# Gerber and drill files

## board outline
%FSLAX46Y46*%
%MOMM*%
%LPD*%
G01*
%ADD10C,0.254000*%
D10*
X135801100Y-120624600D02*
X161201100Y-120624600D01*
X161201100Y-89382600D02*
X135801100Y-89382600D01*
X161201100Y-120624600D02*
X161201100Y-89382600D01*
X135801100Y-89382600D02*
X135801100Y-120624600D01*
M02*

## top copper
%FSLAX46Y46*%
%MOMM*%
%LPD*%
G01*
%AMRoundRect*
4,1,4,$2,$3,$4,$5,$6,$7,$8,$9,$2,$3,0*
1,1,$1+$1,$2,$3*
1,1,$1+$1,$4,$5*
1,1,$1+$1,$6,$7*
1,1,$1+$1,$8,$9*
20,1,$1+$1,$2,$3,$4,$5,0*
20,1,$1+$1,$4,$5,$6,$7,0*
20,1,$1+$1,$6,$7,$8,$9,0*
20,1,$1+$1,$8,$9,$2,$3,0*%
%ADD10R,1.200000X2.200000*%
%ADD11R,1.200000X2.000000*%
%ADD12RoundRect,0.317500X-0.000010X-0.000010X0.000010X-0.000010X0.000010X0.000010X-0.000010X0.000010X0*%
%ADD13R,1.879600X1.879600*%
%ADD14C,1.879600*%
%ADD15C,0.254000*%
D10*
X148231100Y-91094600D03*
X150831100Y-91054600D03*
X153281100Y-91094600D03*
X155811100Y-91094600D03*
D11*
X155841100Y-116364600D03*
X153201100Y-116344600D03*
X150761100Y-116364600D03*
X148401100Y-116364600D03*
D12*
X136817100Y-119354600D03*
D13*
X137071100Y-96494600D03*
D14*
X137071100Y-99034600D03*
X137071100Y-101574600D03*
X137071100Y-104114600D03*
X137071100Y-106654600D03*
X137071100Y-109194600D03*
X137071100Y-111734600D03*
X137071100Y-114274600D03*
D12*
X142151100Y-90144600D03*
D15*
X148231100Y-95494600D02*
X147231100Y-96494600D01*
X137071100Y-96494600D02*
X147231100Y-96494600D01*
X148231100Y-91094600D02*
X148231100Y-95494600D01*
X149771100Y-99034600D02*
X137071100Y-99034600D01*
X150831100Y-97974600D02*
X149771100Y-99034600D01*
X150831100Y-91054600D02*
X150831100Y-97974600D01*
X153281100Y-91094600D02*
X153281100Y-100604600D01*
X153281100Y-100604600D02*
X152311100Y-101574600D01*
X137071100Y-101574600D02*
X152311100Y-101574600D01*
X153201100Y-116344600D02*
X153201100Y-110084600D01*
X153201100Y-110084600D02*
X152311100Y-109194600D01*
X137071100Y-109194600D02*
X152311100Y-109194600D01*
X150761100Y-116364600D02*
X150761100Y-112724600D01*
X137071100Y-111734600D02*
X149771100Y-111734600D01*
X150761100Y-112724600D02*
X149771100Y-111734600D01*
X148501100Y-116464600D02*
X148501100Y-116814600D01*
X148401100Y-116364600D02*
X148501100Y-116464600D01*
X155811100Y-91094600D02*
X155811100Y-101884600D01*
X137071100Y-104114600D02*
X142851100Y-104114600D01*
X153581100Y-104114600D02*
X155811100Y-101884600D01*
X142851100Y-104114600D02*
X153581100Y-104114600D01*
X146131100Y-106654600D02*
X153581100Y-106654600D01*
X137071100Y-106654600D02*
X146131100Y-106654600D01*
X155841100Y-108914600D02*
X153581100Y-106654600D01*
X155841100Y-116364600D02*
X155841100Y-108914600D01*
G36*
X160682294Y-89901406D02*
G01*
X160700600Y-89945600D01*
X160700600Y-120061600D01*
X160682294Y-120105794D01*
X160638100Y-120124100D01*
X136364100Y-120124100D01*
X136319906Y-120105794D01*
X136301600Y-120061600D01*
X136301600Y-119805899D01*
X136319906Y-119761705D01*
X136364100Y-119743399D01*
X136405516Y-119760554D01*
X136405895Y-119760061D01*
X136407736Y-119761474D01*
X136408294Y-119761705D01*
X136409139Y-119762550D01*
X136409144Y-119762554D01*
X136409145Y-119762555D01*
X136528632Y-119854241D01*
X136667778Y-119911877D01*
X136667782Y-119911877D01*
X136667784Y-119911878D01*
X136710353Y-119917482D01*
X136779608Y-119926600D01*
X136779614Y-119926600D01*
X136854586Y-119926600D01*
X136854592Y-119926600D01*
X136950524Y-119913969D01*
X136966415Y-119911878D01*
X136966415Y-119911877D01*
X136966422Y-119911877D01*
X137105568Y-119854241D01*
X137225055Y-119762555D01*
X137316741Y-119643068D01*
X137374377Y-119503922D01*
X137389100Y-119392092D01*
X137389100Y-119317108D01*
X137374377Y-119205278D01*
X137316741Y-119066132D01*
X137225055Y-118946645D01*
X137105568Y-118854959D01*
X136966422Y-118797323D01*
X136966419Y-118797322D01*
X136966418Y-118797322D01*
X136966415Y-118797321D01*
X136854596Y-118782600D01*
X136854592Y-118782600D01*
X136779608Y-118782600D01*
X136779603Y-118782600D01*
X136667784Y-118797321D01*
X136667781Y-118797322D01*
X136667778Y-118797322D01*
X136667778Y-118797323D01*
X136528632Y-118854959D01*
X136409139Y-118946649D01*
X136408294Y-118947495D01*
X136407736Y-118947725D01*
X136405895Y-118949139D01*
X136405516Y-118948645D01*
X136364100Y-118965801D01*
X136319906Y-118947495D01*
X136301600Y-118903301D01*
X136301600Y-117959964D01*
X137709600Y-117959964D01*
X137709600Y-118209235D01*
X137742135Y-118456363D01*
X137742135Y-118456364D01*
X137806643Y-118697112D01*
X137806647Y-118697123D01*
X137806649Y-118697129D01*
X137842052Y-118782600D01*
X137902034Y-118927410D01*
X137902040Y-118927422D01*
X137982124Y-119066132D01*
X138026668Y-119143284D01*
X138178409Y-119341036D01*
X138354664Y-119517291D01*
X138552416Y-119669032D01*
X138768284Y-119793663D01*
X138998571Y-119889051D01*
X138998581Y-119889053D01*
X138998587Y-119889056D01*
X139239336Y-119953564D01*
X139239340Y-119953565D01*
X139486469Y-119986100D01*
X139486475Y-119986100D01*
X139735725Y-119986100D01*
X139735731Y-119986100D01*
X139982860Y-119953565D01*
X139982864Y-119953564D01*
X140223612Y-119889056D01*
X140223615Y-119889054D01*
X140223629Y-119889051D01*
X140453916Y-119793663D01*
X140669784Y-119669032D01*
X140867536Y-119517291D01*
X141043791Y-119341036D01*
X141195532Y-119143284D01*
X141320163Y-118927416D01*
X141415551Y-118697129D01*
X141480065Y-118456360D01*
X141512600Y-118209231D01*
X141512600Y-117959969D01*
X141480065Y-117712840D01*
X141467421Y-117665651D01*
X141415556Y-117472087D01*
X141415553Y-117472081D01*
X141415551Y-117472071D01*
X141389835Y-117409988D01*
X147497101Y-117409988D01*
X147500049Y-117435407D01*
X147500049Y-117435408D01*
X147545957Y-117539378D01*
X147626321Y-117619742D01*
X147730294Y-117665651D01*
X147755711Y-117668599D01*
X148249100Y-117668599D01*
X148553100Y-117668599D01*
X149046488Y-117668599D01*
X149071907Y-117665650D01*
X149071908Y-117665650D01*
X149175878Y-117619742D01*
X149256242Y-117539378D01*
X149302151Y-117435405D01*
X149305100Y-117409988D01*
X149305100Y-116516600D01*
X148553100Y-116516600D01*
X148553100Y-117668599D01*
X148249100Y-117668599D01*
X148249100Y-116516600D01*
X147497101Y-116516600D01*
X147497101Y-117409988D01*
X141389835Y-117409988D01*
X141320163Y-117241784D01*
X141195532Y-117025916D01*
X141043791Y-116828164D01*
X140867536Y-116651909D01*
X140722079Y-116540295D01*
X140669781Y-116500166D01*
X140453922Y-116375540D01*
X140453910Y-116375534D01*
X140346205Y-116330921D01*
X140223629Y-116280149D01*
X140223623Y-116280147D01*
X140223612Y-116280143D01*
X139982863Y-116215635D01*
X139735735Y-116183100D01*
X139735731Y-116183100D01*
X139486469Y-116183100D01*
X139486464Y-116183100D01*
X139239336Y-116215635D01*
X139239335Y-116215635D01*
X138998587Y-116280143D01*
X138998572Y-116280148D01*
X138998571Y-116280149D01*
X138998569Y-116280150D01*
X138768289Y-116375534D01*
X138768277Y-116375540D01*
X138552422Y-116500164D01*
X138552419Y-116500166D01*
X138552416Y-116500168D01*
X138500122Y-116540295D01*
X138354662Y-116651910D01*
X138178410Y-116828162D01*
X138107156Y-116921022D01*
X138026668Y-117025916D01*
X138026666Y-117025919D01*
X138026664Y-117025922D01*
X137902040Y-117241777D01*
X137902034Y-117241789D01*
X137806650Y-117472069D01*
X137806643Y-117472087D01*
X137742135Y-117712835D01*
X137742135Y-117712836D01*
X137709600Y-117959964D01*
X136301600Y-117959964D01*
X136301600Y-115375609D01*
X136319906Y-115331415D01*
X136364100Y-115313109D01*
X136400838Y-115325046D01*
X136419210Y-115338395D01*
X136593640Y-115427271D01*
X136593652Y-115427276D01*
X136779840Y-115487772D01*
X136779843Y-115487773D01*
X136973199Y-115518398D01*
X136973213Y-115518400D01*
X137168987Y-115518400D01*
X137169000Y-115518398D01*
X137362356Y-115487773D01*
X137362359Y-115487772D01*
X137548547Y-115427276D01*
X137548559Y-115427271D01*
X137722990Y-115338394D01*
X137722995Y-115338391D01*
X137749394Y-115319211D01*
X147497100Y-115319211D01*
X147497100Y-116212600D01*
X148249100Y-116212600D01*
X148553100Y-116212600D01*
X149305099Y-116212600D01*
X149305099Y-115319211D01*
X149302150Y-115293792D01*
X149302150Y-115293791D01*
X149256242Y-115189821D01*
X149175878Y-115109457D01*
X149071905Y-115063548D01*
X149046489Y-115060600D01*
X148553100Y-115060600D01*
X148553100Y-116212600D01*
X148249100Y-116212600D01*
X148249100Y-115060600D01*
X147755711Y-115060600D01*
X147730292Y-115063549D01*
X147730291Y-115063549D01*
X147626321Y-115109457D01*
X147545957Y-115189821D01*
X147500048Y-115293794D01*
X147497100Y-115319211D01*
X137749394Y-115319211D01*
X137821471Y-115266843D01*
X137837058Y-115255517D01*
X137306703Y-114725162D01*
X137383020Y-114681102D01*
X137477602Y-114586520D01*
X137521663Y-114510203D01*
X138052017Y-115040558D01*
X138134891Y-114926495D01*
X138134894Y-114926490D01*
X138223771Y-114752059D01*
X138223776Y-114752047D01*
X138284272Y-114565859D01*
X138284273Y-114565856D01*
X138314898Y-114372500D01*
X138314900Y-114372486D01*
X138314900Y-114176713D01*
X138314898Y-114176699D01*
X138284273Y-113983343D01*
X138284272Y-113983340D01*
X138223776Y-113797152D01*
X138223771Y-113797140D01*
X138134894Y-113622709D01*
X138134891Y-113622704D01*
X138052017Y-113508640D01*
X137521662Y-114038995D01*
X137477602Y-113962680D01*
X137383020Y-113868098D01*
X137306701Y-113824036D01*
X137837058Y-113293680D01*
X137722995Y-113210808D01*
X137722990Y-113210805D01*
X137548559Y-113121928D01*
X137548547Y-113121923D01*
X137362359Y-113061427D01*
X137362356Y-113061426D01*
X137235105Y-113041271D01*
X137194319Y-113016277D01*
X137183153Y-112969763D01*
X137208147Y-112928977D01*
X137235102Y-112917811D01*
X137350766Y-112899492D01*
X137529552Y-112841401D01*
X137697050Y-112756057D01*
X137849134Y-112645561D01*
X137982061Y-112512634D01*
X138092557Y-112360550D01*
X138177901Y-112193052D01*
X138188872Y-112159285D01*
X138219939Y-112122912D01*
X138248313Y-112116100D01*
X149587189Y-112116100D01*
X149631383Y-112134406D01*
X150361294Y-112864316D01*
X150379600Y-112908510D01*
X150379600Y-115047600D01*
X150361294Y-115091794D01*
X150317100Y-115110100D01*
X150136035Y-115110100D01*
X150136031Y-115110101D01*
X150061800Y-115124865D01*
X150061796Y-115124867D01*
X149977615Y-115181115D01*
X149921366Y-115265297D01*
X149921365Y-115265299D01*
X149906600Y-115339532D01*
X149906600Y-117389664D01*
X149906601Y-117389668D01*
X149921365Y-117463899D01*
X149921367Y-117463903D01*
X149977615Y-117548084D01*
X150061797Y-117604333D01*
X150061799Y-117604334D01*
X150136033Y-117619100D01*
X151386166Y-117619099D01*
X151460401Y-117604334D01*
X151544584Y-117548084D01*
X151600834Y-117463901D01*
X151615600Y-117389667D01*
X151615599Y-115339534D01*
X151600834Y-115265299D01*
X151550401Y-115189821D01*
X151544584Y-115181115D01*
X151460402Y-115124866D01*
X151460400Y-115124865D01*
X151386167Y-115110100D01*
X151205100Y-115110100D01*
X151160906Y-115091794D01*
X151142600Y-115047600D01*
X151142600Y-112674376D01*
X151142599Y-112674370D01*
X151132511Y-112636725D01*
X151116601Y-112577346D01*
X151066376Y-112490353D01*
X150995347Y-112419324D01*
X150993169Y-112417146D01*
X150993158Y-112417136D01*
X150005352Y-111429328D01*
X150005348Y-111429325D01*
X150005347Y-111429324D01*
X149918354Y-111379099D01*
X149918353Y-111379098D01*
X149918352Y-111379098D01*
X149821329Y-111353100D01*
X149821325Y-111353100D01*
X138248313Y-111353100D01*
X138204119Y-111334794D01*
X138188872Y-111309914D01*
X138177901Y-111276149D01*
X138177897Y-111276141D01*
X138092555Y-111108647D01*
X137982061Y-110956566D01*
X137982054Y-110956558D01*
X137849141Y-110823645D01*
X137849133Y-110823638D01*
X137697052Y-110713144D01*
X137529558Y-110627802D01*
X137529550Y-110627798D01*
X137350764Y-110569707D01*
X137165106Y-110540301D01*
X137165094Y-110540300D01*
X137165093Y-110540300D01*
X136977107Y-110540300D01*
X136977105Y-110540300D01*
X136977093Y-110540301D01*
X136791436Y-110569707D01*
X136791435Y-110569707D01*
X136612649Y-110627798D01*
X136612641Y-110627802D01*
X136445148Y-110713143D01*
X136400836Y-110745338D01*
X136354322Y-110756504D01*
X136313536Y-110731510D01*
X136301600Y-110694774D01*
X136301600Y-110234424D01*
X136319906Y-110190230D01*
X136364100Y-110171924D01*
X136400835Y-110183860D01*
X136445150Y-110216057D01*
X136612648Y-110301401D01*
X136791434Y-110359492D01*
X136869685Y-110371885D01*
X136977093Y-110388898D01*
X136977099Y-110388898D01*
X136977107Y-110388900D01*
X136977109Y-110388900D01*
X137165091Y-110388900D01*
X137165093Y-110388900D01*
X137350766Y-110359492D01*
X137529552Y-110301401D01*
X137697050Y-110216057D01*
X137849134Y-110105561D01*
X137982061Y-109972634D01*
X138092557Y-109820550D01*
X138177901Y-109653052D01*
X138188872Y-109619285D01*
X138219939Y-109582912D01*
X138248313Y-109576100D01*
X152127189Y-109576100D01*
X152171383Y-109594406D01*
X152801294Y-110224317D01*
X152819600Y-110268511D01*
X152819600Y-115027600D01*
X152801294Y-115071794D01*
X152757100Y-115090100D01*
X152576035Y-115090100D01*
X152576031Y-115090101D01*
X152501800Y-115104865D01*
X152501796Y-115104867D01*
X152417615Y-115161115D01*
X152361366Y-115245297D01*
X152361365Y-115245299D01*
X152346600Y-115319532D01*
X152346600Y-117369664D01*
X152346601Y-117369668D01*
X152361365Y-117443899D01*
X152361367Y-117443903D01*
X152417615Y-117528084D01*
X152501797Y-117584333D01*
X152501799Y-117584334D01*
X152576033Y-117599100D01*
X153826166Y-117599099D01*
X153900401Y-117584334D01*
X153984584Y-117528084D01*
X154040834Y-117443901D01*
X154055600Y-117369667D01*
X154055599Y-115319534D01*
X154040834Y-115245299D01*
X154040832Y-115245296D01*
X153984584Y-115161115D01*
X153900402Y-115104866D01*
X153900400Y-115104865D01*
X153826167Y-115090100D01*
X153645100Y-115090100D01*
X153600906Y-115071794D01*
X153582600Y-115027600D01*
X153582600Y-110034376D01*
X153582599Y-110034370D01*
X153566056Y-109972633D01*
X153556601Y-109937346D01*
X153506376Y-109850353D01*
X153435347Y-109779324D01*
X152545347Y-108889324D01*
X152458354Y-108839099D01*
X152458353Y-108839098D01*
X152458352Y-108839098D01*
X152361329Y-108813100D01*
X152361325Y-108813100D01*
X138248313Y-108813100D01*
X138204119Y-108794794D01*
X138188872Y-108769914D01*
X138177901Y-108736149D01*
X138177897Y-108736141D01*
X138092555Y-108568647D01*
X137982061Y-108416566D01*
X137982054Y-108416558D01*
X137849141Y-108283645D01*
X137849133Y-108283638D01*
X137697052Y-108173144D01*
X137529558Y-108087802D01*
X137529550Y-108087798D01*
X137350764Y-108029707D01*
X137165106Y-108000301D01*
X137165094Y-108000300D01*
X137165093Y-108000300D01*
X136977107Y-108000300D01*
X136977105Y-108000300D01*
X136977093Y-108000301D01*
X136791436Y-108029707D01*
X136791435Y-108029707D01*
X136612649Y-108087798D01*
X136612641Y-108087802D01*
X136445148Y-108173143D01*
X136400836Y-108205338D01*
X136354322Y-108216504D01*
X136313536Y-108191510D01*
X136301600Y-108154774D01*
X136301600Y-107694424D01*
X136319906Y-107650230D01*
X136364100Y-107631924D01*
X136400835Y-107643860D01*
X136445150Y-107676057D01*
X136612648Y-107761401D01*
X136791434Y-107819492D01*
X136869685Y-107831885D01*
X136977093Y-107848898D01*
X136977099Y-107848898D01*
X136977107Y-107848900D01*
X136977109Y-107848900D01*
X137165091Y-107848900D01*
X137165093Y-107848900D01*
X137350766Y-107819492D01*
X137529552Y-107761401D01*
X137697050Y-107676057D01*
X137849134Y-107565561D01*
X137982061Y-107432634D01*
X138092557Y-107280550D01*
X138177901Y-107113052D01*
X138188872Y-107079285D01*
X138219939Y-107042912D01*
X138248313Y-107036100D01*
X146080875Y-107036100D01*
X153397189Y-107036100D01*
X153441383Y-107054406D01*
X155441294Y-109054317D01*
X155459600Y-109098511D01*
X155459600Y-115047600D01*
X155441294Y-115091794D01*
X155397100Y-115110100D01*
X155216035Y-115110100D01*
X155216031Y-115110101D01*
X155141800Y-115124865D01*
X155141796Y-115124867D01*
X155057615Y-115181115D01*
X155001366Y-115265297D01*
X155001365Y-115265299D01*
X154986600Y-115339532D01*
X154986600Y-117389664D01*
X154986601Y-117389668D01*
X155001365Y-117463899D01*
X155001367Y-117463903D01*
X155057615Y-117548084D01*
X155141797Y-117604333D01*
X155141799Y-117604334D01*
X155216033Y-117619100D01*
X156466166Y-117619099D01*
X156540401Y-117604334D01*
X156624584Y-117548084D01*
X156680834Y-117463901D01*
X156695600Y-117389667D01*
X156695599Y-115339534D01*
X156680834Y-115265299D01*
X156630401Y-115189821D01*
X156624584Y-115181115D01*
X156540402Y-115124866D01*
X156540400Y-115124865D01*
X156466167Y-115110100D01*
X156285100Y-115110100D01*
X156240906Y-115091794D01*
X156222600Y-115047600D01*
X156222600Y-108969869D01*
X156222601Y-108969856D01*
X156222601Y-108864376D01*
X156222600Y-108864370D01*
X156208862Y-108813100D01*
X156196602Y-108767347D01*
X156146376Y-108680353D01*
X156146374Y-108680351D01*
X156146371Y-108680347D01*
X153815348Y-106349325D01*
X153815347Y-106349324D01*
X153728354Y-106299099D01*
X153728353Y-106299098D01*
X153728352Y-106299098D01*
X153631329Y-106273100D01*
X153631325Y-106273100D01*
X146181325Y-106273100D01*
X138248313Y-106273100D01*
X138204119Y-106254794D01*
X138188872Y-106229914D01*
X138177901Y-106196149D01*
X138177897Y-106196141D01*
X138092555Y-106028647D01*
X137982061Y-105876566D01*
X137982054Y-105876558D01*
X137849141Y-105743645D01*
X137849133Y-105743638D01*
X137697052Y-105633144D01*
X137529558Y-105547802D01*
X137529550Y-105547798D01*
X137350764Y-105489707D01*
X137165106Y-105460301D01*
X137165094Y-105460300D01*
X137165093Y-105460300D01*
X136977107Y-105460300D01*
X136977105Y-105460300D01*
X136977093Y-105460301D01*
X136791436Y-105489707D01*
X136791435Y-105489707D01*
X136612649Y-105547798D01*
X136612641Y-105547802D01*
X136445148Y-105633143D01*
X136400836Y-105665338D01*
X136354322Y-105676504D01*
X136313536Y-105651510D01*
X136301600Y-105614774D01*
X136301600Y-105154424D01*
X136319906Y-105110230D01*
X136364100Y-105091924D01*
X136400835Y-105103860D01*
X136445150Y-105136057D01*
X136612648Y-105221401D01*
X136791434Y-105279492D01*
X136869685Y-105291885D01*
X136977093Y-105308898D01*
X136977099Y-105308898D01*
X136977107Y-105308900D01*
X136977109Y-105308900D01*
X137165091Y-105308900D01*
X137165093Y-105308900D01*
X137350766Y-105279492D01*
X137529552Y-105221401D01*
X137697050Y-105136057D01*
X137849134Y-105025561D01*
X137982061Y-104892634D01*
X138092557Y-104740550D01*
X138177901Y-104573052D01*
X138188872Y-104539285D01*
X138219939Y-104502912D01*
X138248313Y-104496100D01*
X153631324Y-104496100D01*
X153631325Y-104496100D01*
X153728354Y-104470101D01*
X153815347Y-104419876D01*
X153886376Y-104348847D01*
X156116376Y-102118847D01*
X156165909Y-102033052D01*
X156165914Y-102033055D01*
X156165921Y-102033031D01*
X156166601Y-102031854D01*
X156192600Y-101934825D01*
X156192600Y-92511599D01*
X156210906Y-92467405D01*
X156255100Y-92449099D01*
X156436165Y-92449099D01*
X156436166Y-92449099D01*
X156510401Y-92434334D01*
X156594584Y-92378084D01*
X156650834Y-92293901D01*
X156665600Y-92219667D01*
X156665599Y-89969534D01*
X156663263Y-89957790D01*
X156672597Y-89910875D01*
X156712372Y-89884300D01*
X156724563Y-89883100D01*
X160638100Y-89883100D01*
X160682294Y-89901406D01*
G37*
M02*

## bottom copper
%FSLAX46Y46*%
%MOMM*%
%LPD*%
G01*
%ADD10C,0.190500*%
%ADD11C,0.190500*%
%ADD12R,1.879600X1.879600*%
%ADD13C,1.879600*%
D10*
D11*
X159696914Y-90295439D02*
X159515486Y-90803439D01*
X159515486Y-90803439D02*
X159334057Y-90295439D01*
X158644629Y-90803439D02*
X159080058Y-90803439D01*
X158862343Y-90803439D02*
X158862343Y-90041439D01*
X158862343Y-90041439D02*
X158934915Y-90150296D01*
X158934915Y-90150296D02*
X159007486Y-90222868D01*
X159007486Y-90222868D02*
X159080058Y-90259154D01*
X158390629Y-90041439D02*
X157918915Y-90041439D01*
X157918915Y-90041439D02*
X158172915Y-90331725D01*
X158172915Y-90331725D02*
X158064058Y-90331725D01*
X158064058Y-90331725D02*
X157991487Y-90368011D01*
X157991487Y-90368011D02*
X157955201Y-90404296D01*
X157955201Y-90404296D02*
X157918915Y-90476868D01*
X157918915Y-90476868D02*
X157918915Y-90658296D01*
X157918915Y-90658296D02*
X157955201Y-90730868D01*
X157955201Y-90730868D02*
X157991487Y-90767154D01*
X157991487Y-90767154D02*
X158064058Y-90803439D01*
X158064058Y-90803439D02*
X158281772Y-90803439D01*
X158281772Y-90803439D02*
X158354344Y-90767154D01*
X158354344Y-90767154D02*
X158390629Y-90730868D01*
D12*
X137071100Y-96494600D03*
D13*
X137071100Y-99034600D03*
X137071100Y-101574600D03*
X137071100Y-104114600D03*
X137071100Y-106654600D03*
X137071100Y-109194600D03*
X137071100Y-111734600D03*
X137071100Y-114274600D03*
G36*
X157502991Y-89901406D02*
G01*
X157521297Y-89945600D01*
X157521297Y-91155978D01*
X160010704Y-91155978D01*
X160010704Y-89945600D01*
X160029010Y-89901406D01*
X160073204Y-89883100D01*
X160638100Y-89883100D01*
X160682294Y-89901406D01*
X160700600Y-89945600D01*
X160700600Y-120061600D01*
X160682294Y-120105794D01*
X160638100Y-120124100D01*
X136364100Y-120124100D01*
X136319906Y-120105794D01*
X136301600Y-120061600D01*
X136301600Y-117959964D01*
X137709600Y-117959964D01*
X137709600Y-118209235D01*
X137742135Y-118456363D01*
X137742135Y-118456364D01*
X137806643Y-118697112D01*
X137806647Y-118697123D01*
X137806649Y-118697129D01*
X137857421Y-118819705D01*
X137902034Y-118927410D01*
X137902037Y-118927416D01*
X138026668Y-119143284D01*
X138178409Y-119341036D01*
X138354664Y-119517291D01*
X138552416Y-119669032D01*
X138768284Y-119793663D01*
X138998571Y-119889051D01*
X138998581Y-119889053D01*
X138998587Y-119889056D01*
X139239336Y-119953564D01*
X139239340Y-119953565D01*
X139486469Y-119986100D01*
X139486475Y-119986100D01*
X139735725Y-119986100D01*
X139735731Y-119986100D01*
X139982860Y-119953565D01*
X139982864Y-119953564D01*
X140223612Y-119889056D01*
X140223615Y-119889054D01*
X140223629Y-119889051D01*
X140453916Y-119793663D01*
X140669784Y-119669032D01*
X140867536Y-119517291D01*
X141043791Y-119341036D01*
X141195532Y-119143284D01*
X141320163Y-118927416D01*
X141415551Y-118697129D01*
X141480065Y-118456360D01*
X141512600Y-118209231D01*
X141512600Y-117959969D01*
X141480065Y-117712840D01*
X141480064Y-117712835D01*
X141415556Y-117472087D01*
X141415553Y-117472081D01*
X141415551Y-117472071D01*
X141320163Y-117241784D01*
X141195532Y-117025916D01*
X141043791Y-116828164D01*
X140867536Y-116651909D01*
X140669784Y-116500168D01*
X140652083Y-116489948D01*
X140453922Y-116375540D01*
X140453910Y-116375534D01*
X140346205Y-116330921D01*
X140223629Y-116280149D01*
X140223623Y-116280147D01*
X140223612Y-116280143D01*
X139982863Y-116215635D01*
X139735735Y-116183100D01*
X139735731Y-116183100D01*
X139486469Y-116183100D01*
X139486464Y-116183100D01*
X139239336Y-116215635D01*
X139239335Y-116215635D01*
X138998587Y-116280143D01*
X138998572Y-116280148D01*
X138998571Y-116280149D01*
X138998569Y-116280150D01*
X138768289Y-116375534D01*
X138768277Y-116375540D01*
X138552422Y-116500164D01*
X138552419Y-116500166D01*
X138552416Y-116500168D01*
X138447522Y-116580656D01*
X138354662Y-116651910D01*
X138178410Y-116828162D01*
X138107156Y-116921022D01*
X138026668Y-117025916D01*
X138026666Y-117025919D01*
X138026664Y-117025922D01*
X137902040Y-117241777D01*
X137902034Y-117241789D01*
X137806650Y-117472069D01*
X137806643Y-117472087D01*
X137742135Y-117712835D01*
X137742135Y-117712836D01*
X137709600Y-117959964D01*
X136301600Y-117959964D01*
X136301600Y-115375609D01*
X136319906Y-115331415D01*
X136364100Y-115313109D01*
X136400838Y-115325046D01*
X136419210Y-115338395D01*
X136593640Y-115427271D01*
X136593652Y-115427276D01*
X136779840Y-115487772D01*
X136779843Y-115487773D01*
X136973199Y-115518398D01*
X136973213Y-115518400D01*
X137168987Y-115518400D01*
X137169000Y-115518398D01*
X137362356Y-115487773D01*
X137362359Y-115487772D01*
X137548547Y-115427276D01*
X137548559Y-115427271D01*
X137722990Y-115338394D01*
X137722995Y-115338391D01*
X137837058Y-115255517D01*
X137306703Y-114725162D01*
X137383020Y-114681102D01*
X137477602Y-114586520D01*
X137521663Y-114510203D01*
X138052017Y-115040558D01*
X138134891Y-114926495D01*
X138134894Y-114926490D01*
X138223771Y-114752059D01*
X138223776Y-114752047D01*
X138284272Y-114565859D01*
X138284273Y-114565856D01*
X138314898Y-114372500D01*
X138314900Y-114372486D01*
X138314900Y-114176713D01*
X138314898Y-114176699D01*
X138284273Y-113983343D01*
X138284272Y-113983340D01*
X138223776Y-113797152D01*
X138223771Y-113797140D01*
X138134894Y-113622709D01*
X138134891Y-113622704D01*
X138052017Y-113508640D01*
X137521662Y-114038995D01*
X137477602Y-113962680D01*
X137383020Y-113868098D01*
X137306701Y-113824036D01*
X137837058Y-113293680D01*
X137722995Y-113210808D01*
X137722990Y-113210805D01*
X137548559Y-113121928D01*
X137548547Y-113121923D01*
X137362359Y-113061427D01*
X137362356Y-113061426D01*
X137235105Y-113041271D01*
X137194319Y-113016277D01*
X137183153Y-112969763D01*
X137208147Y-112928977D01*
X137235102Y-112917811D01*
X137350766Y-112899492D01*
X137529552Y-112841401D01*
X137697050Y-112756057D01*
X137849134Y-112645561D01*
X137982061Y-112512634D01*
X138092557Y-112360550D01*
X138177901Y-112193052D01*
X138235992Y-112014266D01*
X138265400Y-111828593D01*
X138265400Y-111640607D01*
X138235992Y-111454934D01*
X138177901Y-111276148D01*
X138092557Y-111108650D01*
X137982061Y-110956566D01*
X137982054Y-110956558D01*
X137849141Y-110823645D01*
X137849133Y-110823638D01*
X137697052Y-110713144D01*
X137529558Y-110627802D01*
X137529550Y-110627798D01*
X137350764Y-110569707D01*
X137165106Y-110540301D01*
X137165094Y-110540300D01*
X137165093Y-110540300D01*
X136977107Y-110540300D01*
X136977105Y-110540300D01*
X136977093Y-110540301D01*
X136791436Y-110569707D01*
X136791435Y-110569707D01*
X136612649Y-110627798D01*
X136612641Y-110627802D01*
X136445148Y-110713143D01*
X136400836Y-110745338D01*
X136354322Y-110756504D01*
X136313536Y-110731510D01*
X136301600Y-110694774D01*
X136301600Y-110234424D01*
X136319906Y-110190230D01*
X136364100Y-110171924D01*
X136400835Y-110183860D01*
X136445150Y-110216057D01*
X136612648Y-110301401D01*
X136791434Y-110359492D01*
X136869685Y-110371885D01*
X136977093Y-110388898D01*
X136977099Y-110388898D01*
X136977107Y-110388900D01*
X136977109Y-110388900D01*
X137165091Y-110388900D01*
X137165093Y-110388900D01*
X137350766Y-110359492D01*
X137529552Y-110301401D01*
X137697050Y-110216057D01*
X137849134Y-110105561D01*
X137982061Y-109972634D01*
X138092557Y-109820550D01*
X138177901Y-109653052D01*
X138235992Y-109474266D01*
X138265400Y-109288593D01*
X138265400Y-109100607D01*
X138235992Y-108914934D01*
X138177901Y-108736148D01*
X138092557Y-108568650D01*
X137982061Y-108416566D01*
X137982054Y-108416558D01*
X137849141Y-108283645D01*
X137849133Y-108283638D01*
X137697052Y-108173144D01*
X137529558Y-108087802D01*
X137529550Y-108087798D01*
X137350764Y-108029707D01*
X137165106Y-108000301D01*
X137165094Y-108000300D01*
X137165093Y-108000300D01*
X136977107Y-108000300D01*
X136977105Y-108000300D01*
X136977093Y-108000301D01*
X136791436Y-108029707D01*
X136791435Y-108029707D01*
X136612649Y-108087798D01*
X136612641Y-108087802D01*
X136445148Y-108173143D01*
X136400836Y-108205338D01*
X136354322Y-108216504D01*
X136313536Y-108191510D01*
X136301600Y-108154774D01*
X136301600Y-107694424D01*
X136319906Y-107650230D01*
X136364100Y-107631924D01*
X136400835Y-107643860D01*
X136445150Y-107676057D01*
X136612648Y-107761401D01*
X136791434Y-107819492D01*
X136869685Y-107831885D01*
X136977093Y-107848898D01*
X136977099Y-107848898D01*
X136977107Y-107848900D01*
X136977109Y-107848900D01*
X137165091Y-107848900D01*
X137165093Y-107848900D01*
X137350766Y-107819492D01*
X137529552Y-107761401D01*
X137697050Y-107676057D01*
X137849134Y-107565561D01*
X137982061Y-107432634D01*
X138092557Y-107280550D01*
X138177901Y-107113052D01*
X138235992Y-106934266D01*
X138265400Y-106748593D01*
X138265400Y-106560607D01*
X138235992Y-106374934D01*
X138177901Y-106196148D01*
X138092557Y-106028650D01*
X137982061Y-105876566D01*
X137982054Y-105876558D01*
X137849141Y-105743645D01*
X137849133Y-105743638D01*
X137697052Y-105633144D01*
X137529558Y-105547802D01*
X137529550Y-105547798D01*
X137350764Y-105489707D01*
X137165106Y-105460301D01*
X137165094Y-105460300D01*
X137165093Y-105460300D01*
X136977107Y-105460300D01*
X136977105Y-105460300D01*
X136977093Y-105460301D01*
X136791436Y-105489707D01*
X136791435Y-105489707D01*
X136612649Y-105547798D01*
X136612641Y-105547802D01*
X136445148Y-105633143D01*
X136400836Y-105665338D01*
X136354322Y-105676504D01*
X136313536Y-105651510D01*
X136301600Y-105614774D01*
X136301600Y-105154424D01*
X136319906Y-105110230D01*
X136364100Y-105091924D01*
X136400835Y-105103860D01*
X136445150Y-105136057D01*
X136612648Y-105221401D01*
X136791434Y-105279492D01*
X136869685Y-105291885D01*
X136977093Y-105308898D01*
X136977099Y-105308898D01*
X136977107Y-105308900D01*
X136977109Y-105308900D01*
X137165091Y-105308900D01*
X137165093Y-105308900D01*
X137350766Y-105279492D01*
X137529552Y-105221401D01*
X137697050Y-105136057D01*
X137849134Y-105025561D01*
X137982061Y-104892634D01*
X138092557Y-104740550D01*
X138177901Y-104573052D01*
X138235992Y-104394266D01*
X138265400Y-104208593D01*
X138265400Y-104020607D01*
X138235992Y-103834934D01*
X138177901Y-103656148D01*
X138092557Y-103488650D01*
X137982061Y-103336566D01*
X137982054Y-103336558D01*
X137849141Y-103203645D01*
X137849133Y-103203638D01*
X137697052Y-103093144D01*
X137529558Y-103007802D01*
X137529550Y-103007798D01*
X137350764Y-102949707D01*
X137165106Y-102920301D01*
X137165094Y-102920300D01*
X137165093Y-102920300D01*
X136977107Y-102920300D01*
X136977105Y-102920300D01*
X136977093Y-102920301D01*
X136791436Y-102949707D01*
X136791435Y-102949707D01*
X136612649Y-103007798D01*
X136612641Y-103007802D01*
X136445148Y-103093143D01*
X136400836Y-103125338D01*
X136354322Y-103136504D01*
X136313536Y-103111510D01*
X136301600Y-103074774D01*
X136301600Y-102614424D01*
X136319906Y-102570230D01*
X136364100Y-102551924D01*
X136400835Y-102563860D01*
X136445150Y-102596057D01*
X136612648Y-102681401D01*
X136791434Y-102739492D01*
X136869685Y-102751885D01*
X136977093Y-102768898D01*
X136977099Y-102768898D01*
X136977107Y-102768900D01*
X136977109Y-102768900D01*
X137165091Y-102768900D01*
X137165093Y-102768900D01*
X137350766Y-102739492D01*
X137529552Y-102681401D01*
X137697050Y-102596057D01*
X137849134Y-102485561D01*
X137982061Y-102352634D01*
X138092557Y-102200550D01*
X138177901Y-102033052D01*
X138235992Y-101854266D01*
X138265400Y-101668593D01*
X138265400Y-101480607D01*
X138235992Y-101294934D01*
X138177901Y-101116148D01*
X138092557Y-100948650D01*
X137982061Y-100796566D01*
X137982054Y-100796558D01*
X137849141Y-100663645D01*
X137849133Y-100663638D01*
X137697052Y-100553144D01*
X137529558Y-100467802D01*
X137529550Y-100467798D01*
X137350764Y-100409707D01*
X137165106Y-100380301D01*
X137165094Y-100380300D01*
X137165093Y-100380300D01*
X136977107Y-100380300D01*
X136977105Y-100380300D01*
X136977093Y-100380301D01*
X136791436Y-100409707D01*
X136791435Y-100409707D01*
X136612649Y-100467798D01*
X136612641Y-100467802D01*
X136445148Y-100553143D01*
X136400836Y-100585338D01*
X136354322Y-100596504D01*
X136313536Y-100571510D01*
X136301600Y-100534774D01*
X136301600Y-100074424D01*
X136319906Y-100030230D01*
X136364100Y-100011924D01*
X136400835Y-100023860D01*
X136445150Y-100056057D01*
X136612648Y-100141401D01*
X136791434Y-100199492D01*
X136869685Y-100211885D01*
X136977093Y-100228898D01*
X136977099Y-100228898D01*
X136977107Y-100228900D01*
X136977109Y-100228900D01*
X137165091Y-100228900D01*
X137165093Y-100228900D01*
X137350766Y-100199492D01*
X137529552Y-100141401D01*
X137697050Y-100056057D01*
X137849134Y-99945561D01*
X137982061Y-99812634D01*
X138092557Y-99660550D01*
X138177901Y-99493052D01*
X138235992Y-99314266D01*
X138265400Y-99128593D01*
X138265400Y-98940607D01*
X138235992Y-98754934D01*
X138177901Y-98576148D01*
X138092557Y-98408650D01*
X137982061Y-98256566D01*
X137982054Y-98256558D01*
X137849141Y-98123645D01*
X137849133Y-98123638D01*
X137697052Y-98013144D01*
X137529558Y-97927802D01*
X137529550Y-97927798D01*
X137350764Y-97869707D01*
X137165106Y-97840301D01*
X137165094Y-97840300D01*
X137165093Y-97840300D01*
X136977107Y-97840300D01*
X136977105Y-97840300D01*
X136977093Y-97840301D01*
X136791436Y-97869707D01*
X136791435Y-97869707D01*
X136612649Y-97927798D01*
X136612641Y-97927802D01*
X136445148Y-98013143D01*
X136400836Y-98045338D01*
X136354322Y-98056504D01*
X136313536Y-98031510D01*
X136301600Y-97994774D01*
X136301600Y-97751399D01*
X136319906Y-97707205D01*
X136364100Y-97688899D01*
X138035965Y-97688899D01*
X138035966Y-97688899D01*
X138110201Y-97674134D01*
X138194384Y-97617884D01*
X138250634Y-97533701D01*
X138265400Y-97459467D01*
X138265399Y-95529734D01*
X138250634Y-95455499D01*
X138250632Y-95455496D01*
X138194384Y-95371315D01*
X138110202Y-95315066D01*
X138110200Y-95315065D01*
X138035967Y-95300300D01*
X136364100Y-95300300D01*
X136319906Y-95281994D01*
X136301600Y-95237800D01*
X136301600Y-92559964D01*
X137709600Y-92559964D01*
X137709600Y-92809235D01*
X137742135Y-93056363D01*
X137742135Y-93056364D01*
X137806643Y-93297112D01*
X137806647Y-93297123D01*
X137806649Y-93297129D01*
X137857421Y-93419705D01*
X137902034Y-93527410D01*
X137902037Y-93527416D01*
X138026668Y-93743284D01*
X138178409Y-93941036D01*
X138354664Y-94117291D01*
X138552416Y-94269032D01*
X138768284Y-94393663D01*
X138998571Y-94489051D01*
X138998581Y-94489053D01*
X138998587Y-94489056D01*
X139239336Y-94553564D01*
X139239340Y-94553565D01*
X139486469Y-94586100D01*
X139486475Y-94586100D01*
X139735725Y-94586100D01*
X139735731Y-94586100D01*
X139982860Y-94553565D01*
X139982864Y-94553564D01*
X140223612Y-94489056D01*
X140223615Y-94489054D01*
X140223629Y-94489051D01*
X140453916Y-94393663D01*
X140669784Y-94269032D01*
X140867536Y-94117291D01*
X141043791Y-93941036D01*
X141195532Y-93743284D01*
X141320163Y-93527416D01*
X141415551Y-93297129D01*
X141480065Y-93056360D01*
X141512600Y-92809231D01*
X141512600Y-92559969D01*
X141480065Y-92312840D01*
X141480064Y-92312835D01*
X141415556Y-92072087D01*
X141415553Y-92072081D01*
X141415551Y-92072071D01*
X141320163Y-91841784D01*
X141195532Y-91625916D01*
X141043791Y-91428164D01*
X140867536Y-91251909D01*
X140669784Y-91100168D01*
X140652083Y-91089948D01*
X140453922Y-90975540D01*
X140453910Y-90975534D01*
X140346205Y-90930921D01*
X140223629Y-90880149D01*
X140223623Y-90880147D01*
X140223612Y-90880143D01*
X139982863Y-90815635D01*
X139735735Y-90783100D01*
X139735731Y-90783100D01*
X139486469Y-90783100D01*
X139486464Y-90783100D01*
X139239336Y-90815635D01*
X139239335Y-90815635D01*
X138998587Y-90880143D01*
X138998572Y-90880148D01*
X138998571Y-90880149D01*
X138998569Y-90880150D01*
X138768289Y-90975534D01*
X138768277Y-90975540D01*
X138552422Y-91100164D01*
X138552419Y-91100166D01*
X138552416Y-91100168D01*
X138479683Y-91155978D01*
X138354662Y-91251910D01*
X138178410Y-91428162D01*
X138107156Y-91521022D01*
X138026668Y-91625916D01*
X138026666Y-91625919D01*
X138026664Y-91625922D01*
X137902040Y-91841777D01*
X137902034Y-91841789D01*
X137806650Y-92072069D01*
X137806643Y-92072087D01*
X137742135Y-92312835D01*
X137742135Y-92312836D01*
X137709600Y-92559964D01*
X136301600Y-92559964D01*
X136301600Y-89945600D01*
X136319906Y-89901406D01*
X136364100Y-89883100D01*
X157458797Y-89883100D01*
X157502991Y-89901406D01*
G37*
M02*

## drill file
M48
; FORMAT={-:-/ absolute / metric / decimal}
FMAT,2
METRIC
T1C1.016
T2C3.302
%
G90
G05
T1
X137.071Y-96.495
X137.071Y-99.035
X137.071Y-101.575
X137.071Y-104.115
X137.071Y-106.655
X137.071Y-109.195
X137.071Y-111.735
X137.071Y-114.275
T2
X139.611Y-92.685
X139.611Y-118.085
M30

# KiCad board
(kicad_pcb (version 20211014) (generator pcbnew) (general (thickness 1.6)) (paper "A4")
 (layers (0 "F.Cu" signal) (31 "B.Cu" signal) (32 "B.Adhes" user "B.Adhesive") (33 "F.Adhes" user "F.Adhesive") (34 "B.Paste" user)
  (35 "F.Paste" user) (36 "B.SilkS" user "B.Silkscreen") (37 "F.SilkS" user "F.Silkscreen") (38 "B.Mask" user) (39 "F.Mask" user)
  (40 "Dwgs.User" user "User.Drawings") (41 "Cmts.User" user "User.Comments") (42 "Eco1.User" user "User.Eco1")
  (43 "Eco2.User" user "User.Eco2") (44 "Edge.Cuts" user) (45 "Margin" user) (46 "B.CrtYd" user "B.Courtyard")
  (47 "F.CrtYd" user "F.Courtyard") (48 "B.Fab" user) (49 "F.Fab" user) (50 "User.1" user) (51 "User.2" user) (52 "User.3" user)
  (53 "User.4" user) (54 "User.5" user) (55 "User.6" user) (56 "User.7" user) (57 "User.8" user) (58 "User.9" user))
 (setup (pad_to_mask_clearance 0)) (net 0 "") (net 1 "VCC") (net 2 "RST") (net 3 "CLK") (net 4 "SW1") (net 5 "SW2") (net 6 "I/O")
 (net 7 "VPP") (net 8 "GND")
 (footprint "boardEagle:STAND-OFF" (layer "F.Cu") (at 139.6111 118.0846)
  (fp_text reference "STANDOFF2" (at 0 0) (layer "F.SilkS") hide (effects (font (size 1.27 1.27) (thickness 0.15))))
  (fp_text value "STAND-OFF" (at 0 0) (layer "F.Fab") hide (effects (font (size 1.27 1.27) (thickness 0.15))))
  (pad "" np_thru_hole circle (at 0 0) (size 3.302 3.302) (drill 3.302) (layers *.Cu *.Mask)))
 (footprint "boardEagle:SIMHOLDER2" (layer "F.Cu") (at 143.4211 90.1446 -90)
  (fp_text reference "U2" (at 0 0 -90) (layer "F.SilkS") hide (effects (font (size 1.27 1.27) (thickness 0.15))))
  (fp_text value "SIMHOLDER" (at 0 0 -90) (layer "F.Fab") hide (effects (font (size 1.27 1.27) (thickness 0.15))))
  (pad "1" smd rect (at 0.95 -4.81) (size 1.2 2.2) (layers "F.Cu" "F.Paste" "F.Mask") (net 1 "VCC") (solder_mask_margin 0.1016))
  (pad "2" smd rect (at 0.91 -7.41) (size 1.2 2.2) (layers "F.Cu" "F.Paste" "F.Mask") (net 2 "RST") (solder_mask_margin 0.1016))
  (pad "3" smd rect (at 0.95 -9.86) (size 1.2 2.2) (layers "F.Cu" "F.Paste" "F.Mask") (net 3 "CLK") (solder_mask_margin 0.1016))
  (pad "4" smd rect (at 0.95 -12.39) (size 1.2 2.2) (layers "F.Cu" "F.Paste" "F.Mask") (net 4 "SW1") (solder_mask_margin 0.1016))
  (pad "5" smd rect (at 26.22 -12.42) (size 1.2 2) (layers "F.Cu" "F.Paste" "F.Mask") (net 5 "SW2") (solder_mask_margin 0.1016))
  (pad "6" smd rect (at 26.2 -9.78) (size 1.2 2) (layers "F.Cu" "F.Paste" "F.Mask") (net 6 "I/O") (solder_mask_margin 0.1016))
  (pad "7" smd rect (at 26.22 -7.34) (size 1.2 2) (layers "F.Cu" "F.Paste" "F.Mask") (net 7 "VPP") (solder_mask_margin 0.1016))
  (pad "8" smd rect (at 26.22 -4.98) (size 1.2 2) (layers "F.Cu" "F.Paste" "F.Mask") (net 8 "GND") (solder_mask_margin 0.1016)))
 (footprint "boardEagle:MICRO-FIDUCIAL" (layer "F.Cu") (at 136.8171 119.3546)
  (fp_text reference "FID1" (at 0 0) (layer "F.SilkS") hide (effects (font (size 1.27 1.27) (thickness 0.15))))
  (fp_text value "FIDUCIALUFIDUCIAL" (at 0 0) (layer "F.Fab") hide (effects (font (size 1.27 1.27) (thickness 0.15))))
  (pad "1" smd roundrect (at 0 0) (size 0.635 0.635) (layers "F.Cu" "F.Mask") (roundrect_rratio 0.5) (solder_mask_margin 0.1016)))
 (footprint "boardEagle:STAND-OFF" (layer "F.Cu") (at 139.6111 92.6846)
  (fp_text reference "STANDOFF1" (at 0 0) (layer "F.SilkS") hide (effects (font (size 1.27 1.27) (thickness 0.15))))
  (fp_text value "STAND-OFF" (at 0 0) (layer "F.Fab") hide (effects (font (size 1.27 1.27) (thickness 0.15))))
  (pad "" np_thru_hole circle (at 0 0) (size 3.302 3.302) (drill 3.302) (layers *.Cu *.Mask)))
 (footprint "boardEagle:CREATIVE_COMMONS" (layer "F.Cu") (at 116.7511 130.7846)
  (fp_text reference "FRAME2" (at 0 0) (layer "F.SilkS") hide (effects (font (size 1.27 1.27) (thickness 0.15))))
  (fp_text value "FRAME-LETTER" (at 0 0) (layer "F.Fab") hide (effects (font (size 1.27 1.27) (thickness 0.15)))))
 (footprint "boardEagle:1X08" (layer "F.Cu") (at 137.0711 96.4946 -90)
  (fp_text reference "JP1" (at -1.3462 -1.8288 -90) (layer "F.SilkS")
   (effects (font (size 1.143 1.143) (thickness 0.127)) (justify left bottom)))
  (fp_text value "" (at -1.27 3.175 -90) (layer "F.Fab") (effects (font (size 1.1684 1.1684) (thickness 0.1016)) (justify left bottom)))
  (pad "1" thru_hole rect (at 0 0) (size 1.8796 1.8796) (drill 1.016) (layers *.Cu *.Mask) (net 1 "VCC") (solder_mask_margin 0.1016))
  (pad "2" thru_hole circle (at 2.54 0) (size 1.8796 1.8796) (drill 1.016) (layers *.Cu *.Mask) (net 2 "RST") (solder_mask_margin 0.1016))
  (pad "3" thru_hole circle (at 5.08 0) (size 1.8796 1.8796) (drill 1.016) (layers *.Cu *.Mask) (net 3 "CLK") (solder_mask_margin 0.1016))
  (pad "4" thru_hole circle (at 7.62 0) (size 1.8796 1.8796) (drill 1.016) (layers *.Cu *.Mask) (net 4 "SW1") (solder_mask_margin 0.1016))
  (pad "5" thru_hole circle (at 10.16 0) (size 1.8796 1.8796) (drill 1.016) (layers *.Cu *.Mask) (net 5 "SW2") (solder_mask_margin 0.1016))
  (pad "6" thru_hole circle (at 12.7 0) (size 1.8796 1.8796) (drill 1.016) (layers *.Cu *.Mask) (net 6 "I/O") (solder_mask_margin 0.1016))
  (pad "7" thru_hole circle (at 15.24 0) (size 1.8796 1.8796) (drill 1.016) (layers *.Cu *.Mask) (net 7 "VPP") (solder_mask_margin 0.1016))
  (pad "8" thru_hole circle (at 17.78 0) (size 1.8796 1.8796) (drill 1.016) (layers *.Cu *.Mask) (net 8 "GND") (solder_mask_margin 0.1016)))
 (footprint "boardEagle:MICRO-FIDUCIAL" (layer "F.Cu") (at 142.1511 90.1446)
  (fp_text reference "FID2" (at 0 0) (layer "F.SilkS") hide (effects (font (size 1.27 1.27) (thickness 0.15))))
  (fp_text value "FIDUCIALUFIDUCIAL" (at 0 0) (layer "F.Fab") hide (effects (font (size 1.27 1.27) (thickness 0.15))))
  (pad "1" smd roundrect (at 0 0) (size 0.635 0.635) (layers "F.Cu" "F.Mask") (roundrect_rratio 0.5) (solder_mask_margin 0.1016)))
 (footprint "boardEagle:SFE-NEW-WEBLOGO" (layer "B.Cu") (at 150.4061 115.0366 90)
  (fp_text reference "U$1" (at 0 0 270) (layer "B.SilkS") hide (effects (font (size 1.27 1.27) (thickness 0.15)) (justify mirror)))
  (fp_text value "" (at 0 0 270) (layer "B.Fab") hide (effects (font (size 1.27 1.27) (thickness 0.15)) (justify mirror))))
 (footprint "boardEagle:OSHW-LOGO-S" (layer "B.Cu") (at 158.6611 118.0846 90)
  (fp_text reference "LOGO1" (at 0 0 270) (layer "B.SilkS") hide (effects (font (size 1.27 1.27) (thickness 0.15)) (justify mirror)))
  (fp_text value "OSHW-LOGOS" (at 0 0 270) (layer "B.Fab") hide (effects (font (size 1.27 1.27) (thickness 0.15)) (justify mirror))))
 (gr_line (start 135.8011 120.6246) (end 161.2011 120.6246) (layer "Edge.Cuts") (width 0.254))
 (gr_line (start 161.2011 89.3826) (end 135.8011 89.3826) (layer "Edge.Cuts") (width 0.254))
 (gr_line (start 161.2011 120.6246) (end 161.2011 89.3826) (layer "Edge.Cuts") (width 0.254))
 (gr_line (start 135.8011 89.3826) (end 135.8011 120.6246) (layer "Edge.Cuts") (width 0.254))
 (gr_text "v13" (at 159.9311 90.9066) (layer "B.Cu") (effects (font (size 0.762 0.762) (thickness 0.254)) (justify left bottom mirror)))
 (segment (start 148.2311 95.4946) (end 147.2311 96.4946) (width 0.254) (layer "F.Cu") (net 1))
 (segment (start 137.0711 96.4946) (end 147.2311 96.4946) (width 0.254) (layer "F.Cu") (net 1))
 (segment (start 148.2311 91.0946) (end 148.2311 95.4946) (width 0.254) (layer "F.Cu") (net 1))
 (segment (start 149.7711 99.0346) (end 137.0711 99.0346) (width 0.254) (layer "F.Cu") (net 2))
 (segment (start 150.8311 97.9746) (end 149.7711 99.0346) (width 0.254) (layer "F.Cu") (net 2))
 (segment (start 150.8311 91.0546) (end 150.8311 97.9746) (width 0.254) (layer "F.Cu") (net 2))
 (segment (start 153.2811 91.0946) (end 153.2811 100.6046) (width 0.254) (layer "F.Cu") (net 3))
 (segment (start 153.2811 100.6046) (end 152.3111 101.5746) (width 0.254) (layer "F.Cu") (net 3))
 (segment (start 137.0711 101.5746) (end 152.3111 101.5746) (width 0.254) (layer "F.Cu") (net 3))
 (segment (start 153.2011 116.3446) (end 153.2011 110.0846) (width 0.254) (layer "F.Cu") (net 6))
 (segment (start 153.2011 110.0846) (end 152.3111 109.1946) (width 0.254) (layer "F.Cu") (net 6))
 (segment (start 137.0711 109.1946) (end 152.3111 109.1946) (width 0.254) (layer "F.Cu") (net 6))
 (segment (start 150.7611 116.3646) (end 150.7611 112.7246) (width 0.254) (layer "F.Cu") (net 7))
 (segment (start 137.0711 111.7346) (end 149.7711 111.7346) (width 0.254) (layer "F.Cu") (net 7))
 (segment (start 150.7611 112.7246) (end 149.7711 111.7346) (width 0.254) (layer "F.Cu") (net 7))
 (segment (start 148.5011 116.4646) (end 148.5011 116.8146) (width 0.254) (layer "F.Cu") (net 8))
 (segment (start 148.4011 116.3646) (end 148.5011 116.4646) (width 0.254) (layer "F.Cu") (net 8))
 (segment (start 155.8111 91.0946) (end 155.8111 101.8846) (width 0.254) (layer "F.Cu") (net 4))
 (segment (start 137.0711 104.1146) (end 142.8511 104.1146) (width 0.254) (layer "F.Cu") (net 4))
 (segment (start 153.5811 104.1146) (end 155.8111 101.8846) (width 0.254) (layer "F.Cu") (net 4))
 (segment (start 142.8511 104.1146) (end 153.5811 104.1146) (width 0.254) (layer "F.Cu") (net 4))
 (segment (start 146.1311 106.6546) (end 153.5811 106.6546) (width 0.254) (layer "F.Cu") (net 5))
 (segment (start 137.0711 106.6546) (end 146.1311 106.6546) (width 0.254) (layer "F.Cu") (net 5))
 (segment (start 155.8411 108.9146) (end 153.5811 106.6546) (width 0.254) (layer "F.Cu") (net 5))
 (segment (start 155.8411 116.3646) (end 155.8411 108.9146) (width 0.254) (layer "F.Cu") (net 5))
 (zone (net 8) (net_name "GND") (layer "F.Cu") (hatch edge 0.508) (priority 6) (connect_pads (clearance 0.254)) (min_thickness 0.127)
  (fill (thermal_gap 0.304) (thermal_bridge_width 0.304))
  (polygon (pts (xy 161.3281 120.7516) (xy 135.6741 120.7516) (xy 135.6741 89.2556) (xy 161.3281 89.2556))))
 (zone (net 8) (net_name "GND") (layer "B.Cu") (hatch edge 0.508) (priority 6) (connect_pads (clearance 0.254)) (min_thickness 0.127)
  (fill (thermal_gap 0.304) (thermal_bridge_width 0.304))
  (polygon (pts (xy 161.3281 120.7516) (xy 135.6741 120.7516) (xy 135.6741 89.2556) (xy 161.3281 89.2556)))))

